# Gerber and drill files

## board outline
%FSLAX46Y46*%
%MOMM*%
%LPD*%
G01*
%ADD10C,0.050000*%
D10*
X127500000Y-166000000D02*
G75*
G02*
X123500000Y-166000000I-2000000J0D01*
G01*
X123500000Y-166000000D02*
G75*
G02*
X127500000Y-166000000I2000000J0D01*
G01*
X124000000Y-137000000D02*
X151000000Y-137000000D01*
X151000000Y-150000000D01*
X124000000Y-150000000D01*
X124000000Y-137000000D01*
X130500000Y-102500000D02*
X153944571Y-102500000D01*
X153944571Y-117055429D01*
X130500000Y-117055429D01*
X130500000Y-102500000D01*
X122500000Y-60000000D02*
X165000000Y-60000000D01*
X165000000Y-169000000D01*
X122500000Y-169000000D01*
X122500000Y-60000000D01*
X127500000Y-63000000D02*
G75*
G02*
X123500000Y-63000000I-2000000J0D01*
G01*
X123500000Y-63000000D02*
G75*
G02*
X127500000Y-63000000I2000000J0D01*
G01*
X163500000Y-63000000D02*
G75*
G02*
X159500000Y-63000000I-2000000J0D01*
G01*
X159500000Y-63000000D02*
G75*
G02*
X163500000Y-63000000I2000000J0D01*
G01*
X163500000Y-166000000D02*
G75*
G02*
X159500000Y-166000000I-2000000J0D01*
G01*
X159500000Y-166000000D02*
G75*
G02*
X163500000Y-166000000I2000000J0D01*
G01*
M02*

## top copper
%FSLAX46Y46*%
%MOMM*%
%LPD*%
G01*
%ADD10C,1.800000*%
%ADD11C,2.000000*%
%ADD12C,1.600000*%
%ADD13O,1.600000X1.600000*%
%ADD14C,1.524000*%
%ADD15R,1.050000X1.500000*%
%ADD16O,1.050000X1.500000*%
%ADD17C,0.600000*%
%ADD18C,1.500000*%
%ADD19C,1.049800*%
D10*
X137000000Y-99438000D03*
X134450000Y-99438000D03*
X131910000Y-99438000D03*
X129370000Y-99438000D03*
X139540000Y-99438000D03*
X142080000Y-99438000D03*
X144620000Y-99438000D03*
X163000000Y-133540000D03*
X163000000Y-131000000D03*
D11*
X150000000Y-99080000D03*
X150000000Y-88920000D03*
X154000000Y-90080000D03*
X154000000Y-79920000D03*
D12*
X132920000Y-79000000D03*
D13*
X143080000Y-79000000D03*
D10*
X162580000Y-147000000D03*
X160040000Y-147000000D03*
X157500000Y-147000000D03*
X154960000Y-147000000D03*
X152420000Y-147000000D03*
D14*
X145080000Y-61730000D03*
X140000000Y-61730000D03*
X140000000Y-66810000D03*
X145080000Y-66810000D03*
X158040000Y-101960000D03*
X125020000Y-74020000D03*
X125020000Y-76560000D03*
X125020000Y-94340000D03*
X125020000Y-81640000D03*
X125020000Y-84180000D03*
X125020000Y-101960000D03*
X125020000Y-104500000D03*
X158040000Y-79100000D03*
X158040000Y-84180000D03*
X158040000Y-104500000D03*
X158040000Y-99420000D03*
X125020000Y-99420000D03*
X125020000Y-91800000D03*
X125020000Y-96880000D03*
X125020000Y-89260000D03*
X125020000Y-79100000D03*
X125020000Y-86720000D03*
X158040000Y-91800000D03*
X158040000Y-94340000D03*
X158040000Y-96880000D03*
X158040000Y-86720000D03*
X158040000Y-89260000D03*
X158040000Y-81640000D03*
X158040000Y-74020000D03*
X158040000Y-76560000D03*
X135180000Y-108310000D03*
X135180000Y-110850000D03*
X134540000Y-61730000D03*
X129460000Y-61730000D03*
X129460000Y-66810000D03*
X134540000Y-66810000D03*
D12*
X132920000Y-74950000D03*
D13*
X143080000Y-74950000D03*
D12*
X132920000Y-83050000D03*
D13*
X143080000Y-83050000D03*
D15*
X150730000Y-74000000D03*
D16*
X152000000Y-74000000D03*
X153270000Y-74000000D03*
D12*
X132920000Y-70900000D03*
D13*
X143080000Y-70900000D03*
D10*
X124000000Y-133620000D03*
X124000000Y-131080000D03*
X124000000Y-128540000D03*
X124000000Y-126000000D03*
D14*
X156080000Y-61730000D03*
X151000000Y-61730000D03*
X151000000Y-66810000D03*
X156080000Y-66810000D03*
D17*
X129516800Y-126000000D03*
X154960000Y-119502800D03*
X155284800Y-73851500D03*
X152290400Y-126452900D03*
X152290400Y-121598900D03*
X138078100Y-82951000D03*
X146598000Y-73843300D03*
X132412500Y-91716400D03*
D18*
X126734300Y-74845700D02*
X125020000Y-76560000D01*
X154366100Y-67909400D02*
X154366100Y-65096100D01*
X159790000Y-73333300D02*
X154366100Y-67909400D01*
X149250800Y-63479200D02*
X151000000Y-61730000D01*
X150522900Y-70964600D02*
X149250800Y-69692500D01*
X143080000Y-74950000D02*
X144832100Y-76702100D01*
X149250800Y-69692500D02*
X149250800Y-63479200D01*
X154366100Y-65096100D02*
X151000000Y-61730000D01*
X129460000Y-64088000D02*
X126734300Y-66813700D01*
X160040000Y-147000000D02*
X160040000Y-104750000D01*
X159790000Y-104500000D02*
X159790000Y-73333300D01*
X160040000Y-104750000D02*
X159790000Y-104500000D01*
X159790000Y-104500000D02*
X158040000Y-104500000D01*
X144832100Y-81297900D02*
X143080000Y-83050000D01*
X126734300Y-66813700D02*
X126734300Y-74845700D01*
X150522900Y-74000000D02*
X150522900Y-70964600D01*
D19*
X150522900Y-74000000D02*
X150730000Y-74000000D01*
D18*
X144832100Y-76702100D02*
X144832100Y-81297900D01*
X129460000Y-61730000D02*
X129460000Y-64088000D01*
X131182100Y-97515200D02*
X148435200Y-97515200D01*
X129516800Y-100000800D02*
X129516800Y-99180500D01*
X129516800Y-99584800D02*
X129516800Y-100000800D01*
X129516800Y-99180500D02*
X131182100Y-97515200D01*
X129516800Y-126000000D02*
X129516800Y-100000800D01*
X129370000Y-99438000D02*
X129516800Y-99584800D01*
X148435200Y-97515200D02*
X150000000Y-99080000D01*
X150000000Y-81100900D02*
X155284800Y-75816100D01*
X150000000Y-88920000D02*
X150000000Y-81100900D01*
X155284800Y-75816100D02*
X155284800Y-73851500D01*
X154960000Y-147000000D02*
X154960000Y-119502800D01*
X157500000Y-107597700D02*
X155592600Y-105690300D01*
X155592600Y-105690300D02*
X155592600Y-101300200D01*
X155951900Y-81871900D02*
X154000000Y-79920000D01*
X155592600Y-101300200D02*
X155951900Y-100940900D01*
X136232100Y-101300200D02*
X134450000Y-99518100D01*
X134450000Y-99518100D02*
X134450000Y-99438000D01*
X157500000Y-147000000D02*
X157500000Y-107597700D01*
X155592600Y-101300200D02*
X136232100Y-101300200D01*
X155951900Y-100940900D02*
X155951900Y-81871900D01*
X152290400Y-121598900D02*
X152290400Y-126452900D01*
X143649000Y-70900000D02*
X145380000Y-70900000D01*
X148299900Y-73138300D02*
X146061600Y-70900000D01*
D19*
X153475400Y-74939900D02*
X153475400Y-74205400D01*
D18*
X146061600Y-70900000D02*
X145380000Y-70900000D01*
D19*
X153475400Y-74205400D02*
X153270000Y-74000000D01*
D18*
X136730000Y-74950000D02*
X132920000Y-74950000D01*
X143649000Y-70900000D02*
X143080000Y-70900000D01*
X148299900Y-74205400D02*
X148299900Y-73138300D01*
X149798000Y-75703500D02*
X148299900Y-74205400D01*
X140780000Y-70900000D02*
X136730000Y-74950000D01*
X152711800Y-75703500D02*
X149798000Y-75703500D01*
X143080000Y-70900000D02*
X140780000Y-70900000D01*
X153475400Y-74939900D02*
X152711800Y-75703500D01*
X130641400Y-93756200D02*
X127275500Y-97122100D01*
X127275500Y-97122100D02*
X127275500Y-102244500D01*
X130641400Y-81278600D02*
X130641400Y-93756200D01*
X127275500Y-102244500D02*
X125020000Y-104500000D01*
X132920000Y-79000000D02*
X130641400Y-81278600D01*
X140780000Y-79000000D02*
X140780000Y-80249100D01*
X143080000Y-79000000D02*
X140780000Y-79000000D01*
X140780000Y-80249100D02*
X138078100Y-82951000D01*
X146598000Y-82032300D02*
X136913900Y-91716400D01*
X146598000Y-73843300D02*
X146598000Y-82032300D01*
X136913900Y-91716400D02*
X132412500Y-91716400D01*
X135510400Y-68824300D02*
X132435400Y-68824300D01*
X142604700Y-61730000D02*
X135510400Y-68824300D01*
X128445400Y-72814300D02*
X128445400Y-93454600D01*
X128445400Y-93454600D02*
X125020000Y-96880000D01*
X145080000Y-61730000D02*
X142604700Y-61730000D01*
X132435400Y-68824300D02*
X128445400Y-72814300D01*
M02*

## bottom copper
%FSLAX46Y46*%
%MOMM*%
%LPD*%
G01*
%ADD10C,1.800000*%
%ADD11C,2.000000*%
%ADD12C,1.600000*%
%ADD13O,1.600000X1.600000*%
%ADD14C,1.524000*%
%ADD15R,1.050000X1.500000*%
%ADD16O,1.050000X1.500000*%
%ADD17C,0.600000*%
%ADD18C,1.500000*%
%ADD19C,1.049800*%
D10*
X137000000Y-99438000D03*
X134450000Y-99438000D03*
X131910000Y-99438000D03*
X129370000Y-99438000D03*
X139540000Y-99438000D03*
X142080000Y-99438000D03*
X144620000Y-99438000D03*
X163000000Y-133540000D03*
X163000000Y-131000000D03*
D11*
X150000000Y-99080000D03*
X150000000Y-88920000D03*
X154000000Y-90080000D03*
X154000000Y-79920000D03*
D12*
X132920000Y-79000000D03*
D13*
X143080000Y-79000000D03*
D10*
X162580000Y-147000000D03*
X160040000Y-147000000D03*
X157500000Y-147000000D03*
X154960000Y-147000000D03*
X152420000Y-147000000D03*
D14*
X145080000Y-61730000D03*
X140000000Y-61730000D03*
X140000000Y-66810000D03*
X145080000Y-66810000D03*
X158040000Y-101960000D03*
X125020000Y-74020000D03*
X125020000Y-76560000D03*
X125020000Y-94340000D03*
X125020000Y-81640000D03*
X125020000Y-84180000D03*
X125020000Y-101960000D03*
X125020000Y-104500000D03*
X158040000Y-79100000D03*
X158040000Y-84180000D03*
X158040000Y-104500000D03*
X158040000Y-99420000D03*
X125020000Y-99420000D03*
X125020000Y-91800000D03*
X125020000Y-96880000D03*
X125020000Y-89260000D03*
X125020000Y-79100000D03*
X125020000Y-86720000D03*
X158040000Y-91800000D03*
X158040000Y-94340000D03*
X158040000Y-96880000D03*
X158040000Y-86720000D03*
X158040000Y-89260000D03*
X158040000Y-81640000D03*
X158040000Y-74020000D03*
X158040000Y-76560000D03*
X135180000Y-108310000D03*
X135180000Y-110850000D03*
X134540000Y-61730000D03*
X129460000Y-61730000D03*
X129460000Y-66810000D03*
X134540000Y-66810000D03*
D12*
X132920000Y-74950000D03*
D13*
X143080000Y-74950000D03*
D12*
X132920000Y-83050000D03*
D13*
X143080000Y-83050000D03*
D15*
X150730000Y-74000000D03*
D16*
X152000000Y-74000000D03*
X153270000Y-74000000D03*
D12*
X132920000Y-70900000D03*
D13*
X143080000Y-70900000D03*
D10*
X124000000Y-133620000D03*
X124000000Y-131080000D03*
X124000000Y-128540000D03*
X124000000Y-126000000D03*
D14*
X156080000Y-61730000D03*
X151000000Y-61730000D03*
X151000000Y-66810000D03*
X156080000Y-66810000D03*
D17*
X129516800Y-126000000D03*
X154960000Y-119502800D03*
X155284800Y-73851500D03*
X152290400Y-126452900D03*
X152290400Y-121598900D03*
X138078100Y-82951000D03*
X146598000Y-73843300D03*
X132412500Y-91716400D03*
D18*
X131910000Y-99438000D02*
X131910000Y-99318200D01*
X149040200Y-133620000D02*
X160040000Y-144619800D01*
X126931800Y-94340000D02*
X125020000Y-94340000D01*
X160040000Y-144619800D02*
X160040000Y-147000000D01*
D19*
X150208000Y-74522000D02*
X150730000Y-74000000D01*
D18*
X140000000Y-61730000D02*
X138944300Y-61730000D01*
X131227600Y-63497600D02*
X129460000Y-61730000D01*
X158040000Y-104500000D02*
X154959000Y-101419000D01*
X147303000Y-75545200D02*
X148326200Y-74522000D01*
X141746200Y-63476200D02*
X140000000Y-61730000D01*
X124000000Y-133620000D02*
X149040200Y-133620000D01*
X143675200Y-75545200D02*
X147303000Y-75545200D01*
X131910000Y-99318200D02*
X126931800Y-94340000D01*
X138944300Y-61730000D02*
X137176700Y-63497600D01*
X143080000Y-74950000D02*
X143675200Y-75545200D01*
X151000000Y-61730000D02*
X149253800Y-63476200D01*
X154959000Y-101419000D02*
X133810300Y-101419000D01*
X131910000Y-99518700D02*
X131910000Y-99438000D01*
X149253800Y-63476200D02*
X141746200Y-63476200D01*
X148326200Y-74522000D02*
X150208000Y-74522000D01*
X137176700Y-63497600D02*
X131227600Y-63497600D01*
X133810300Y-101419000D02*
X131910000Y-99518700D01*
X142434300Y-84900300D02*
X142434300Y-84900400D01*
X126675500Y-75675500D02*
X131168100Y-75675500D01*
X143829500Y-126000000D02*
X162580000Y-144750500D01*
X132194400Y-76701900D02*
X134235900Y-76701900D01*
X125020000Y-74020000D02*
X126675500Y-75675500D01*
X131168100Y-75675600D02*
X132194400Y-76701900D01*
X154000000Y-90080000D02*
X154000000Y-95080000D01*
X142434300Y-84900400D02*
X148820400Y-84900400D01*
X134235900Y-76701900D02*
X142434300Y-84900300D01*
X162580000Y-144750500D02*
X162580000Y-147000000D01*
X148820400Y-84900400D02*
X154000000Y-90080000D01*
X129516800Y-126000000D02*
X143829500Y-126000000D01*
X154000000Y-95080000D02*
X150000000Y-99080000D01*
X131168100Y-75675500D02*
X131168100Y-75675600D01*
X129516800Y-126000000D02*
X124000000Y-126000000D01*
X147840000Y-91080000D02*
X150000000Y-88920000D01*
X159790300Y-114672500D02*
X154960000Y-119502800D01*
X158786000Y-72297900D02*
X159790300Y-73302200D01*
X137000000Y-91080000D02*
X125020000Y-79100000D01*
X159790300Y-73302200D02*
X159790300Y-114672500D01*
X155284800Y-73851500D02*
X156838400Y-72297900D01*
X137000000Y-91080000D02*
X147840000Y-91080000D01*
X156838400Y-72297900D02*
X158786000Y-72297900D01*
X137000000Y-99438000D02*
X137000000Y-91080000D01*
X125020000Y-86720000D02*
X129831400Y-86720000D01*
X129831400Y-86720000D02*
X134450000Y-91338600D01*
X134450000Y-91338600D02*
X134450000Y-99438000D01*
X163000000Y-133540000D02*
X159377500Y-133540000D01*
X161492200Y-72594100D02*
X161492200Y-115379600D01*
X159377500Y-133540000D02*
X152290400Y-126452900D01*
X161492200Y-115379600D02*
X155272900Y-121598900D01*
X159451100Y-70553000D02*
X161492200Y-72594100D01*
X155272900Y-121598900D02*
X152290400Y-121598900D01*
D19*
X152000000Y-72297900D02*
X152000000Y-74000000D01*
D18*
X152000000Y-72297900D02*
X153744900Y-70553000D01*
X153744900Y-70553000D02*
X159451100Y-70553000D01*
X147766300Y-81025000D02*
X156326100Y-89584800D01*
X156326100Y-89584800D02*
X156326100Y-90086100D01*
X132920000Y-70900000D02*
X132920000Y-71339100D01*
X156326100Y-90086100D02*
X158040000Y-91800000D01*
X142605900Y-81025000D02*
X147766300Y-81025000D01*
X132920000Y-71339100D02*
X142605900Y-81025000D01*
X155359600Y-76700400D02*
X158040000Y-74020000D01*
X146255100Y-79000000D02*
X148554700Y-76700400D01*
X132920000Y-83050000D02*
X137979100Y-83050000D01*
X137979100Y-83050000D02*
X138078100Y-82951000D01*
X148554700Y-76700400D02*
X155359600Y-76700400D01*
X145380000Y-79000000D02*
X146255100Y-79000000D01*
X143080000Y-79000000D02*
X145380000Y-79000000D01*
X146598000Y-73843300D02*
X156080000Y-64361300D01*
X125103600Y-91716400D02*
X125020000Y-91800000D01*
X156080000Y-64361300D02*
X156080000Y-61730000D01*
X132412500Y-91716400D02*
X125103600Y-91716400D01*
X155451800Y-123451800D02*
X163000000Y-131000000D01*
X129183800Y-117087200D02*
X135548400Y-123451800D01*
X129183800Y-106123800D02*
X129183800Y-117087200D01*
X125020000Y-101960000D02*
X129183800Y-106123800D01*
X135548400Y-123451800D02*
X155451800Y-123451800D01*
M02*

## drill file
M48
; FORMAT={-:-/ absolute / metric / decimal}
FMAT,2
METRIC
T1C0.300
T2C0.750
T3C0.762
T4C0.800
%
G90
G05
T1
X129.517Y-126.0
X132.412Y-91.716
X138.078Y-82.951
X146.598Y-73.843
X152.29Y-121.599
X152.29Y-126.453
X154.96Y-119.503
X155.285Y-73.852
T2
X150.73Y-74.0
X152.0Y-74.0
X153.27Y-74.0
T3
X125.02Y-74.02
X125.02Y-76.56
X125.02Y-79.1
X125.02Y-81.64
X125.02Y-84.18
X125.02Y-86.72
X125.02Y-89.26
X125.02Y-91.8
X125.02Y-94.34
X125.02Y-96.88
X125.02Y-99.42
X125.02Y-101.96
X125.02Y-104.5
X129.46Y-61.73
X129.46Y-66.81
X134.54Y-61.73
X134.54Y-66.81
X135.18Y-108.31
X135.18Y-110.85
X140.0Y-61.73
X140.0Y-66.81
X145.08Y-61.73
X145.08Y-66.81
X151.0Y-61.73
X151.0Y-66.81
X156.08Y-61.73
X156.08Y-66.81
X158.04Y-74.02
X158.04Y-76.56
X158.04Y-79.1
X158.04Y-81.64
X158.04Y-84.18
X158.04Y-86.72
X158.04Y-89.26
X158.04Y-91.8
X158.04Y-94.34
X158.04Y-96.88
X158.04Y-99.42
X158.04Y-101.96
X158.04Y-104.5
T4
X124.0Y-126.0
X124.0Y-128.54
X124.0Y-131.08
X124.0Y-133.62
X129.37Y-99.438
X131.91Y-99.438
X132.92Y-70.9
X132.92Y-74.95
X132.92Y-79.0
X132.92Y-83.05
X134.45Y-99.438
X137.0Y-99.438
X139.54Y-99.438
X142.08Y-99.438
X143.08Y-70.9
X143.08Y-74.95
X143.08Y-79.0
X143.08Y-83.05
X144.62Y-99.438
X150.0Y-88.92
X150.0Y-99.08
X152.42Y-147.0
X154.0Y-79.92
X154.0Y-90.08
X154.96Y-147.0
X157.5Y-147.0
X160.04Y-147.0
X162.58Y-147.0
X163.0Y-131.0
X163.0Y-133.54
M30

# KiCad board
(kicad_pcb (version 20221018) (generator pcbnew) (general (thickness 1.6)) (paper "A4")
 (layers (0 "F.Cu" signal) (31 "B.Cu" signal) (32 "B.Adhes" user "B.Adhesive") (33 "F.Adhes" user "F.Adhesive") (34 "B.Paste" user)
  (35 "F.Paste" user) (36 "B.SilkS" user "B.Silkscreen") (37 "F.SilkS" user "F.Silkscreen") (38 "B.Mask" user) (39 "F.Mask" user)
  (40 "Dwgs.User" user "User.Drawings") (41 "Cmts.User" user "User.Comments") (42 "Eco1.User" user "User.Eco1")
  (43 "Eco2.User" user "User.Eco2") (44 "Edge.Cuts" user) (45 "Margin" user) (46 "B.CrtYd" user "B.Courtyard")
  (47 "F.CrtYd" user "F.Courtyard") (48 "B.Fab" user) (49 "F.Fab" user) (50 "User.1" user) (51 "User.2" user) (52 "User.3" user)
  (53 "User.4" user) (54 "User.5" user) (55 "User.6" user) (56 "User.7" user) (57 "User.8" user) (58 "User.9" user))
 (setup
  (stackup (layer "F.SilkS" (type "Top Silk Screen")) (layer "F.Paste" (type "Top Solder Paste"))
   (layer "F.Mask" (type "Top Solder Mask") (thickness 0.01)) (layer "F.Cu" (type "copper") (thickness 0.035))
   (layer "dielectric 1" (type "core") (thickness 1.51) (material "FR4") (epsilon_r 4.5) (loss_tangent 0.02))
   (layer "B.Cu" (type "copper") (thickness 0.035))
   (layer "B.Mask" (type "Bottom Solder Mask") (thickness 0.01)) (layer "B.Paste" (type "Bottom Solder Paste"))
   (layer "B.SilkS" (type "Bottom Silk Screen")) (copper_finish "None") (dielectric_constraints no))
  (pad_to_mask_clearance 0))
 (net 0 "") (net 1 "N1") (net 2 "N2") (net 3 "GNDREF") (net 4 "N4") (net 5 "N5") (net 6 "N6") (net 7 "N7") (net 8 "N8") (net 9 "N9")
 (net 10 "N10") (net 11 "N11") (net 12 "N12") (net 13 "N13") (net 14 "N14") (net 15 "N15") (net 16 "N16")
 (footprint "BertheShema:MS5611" (layer "F.Cu") (at 133.19 96.898)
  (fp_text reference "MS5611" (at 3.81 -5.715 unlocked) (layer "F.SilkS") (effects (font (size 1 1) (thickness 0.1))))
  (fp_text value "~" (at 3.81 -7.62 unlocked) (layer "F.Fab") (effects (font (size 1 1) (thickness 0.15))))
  (pad "1" thru_hole circle (at 3.81 2.54) (size 1.8 1.8) (drill 0.8) (layers "*.Cu" "*.Mask") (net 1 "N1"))
  (pad "2" thru_hole circle (at 1.26 2.54) (size 1.8 1.8) (drill 0.8) (layers "*.Cu" "*.Mask") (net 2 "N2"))
  (pad "3" thru_hole circle (at -1.28 2.54) (size 1.8 1.8) (drill 0.8) (layers "*.Cu" "*.Mask") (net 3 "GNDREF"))
  (pad "4" thru_hole circle (at -3.82 2.54) (size 1.8 1.8) (drill 0.8) (layers "*.Cu" "*.Mask") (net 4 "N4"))
  (pad "5" thru_hole circle (at 6.35 2.54) (size 1.8 1.8) (drill 0.8) (layers "*.Cu" "*.Mask"))
  (pad "6" thru_hole circle (at 8.89 2.54) (size 1.8 1.8) (drill 0.8) (layers "*.Cu" "*.Mask"))
  (pad "7" thru_hole circle (at 11.43 2.54) (size 1.8 1.8) (drill 0.8) (layers "*.Cu" "*.Mask")))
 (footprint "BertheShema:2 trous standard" (layer "F.Cu") (at 163 133.54)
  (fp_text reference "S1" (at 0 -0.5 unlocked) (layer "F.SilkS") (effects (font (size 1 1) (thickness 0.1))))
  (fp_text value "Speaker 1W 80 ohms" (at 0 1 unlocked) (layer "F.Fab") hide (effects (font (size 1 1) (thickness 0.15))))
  (pad "1" thru_hole circle (at 0 0) (size 1.8 1.8) (drill 0.8) (layers "*.Cu" "*.Mask") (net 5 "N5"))
  (pad "2" thru_hole circle (at 0 -2.54) (size 1.8 1.8) (drill 0.8) (layers "*.Cu" "*.Mask") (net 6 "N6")))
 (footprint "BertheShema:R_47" (layer "F.Cu") (at 150 94 -90)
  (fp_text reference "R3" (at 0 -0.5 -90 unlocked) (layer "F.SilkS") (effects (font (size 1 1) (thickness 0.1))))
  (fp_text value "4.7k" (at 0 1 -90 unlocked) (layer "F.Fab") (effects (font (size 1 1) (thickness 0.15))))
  (pad "1" thru_hole circle (at 5.08 0 270) (size 2 2) (drill 0.8) (layers "*.Cu" "*.Mask") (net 4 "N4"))
  (pad "2" thru_hole circle (at -5.08 0 270) (size 2 2) (drill 0.8) (layers "*.Cu" "*.Mask") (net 1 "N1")))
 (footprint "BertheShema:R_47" (layer "F.Cu") (at 154 85 -90)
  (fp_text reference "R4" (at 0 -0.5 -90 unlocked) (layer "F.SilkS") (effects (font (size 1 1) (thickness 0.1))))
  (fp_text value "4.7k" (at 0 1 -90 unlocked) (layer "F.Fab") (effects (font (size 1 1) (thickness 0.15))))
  (pad "1" thru_hole circle (at 5.08 0 270) (size 2 2) (drill 0.8) (layers "*.Cu" "*.Mask") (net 4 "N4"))
  (pad "2" thru_hole circle (at -5.08 0 270) (size 2 2) (drill 0.8) (layers "*.Cu" "*.Mask") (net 2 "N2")))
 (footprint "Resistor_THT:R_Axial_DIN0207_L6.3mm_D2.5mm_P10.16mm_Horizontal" (layer "F.Cu") (at 132.92 79)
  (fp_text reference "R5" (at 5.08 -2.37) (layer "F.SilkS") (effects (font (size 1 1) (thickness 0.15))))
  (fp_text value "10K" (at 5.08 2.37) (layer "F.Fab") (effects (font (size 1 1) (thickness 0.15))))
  (pad "1" thru_hole circle (at 0 0) (size 1.6 1.6) (drill 0.8) (layers "*.Cu" "*.Mask") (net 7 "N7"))
  (pad "2" thru_hole oval (at 10.16 0) (size 1.6 1.6) (drill 0.8) (layers "*.Cu" "*.Mask") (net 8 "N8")))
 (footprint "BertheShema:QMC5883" (layer "F.Cu") (at 157.54 153 180)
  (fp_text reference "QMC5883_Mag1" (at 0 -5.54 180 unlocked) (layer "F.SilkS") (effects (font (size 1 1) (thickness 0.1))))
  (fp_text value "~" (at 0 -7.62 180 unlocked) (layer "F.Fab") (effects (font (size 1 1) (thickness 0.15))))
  (pad "1" thru_hole circle (at -5.04 6 180) (size 1.8 1.8) (drill 0.8) (layers "*.Cu" "*.Mask") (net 4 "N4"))
  (pad "2" thru_hole circle (at -2.5 6 180) (size 1.8 1.8) (drill 0.8) (layers "*.Cu" "*.Mask") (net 3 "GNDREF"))
  (pad "3" thru_hole circle (at 0.04 6 180) (size 1.8 1.8) (drill 0.8) (layers "*.Cu" "*.Mask") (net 2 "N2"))
  (pad "4" thru_hole circle (at 2.58 6 180) (size 1.8 1.8) (drill 0.8) (layers "*.Cu" "*.Mask") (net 1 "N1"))
  (pad "5" thru_hole circle (at 5.12 6 180) (size 1.8 1.8) (drill 0.8) (layers "*.Cu" "*.Mask")))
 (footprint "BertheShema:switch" (layer "F.Cu") (at 142.54 63)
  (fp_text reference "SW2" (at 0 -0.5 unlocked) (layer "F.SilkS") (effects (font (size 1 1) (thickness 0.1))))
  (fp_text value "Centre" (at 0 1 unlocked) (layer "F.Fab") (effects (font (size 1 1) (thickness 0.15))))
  (pad "1" thru_hole circle (at 2.54 -1.27) (size 1.524 1.524) (drill 0.762) (layers "*.Cu" "*.Mask") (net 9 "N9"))
  (pad "2" thru_hole circle (at -2.54 -1.27) (size 1.524 1.524) (drill 0.762) (layers "*.Cu" "*.Mask") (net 3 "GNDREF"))
  (pad "3" thru_hole circle (at -2.54 3.81) (size 1.524 1.524) (drill 0.762) (layers "*.Cu" "*.Mask"))
  (pad "4" thru_hole circle (at 2.54 3.81) (size 1.524 1.524) (drill 0.762) (layers "*.Cu" "*.Mask")))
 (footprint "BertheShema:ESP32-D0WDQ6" (layer "F.Cu") (at 140.26 89.26)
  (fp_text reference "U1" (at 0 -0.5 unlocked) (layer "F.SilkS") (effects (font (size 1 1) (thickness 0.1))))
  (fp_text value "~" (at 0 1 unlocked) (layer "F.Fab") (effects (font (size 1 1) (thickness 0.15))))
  (pad "0" thru_hole circle (at 17.78 12.7) (size 1.524 1.524) (drill 0.762) (layers "*.Cu" "*.Mask"))
  (pad "1" thru_hole circle (at -15.24 -15.24) (size 1.524 1.524) (drill 0.762) (layers "*.Cu" "*.Mask") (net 4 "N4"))
  (pad "2" thru_hole circle (at -15.24 -12.7) (size 1.524 1.524) (drill 0.762) (layers "*.Cu" "*.Mask") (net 3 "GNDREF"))
  (pad "2" thru_hole circle (at -15.24 5.08) (size 1.524 1.524) (drill 0.762) (layers "*.Cu" "*.Mask") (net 3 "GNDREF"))
  (pad "3" thru_hole circle (at -15.24 -7.62) (size 1.524 1.524) (drill 0.762) (layers "*.Cu" "*.Mask") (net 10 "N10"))
  (pad "4" thru_hole circle (at -15.24 -5.08) (size 1.524 1.524) (drill 0.762) (layers "*.Cu" "*.Mask") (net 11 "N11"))
  (pad "5" thru_hole circle (at -15.24 12.7) (size 1.524 1.524) (drill 0.762) (layers "*.Cu" "*.Mask") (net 6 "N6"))
  (pad "6" thru_hole circle (at -15.24 15.24) (size 1.524 1.524) (drill 0.762) (layers "*.Cu" "*.Mask") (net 7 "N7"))
  (pad "7" thru_hole circle (at 17.78 -10.16) (size 1.524 1.524) (drill 0.762) (layers "*.Cu" "*.Mask"))
  (pad "8" thru_hole circle (at 17.78 -5.08) (size 1.524 1.524) (drill 0.762) (layers "*.Cu" "*.Mask"))
  (pad "9" thru_hole circle (at 17.78 15.24) (size 1.524 1.524) (drill 0.762) (layers "*.Cu" "*.Mask") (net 3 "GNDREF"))
  (pad "12" thru_hole circle (at 17.78 10.16) (size 1.524 1.524) (drill 0.762) (layers "*.Cu" "*.Mask"))
  (pad "13" thru_hole circle (at -15.24 10.16) (size 1.524 1.524) (drill 0.762) (layers "*.Cu" "*.Mask") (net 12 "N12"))
  (pad "14" thru_hole circle (at -15.24 2.54) (size 1.524 1.524) (drill 0.762) (layers "*.Cu" "*.Mask") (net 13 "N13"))
  (pad "15" thru_hole circle (at -15.24 7.62) (size 1.524 1.524) (drill 0.762) (layers "*.Cu" "*.Mask") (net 9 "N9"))
  (pad "19" thru_hole circle (at -15.24 0) (size 1.524 1.524) (drill 0.762) (layers "*.Cu" "*.Mask"))
  (pad "21" thru_hole circle (at -15.24 -10.16) (size 1.524 1.524) (drill 0.762) (layers "*.Cu" "*.Mask") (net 1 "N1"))
  (pad "22" thru_hole circle (at -15.24 -2.54) (size 1.524 1.524) (drill 0.762) (layers "*.Cu" "*.Mask") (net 2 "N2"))
  (pad "25" thru_hole circle (at 17.78 2.54) (size 1.524 1.524) (drill 0.762) (layers "*.Cu" "*.Mask") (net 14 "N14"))
  (pad "26" thru_hole circle (at 17.78 5.08) (size 1.524 1.524) (drill 0.762) (layers "*.Cu" "*.Mask"))
  (pad "27" thru_hole circle (at 17.78 7.62) (size 1.524 1.524) (drill 0.762) (layers "*.Cu" "*.Mask"))
  (pad "32" thru_hole circle (at 17.78 -2.54) (size 1.524 1.524) (drill 0.762) (layers "*.Cu" "*.Mask"))
  (pad "33" thru_hole circle (at 17.78 0) (size 1.524 1.524) (drill 0.762) (layers "*.Cu" "*.Mask"))
  (pad "34" thru_hole circle (at 17.78 -7.62) (size 1.524 1.524) (drill 0.762) (layers "*.Cu" "*.Mask"))
  (pad "36" thru_hole circle (at 17.78 -15.24) (size 1.524 1.524) (drill 0.762) (layers "*.Cu" "*.Mask") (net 8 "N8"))
  (pad "39" thru_hole circle (at 17.78 -12.7) (size 1.524 1.524) (drill 0.762) (layers "*.Cu" "*.Mask"))
  (pad "40" thru_hole circle (at -5.08 19.05) (size 1.524 1.524) (drill 0.762) (layers "*.Cu" "*.Mask"))
  (pad "41" thru_hole circle (at -5.08 21.59) (size 1.524 1.524) (drill 0.762) (layers "*.Cu" "*.Mask")))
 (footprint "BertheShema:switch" (layer "F.Cu") (at 132 63)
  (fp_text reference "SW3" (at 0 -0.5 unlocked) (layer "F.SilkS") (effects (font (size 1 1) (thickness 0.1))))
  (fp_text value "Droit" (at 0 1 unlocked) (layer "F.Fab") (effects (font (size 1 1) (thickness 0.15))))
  (pad "1" thru_hole circle (at 2.54 -1.27) (size 1.524 1.524) (drill 0.762) (layers "*.Cu" "*.Mask") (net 12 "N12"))
  (pad "2" thru_hole circle (at -2.54 -1.27) (size 1.524 1.524) (drill 0.762) (layers "*.Cu" "*.Mask") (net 3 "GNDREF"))
  (pad "3" thru_hole circle (at -2.54 3.81) (size 1.524 1.524) (drill 0.762) (layers "*.Cu" "*.Mask"))
  (pad "4" thru_hole circle (at 2.54 3.81) (size 1.524 1.524) (drill 0.762) (layers "*.Cu" "*.Mask")))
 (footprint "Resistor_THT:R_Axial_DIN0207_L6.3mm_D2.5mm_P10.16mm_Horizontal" (layer "F.Cu") (at 132.92 74.95)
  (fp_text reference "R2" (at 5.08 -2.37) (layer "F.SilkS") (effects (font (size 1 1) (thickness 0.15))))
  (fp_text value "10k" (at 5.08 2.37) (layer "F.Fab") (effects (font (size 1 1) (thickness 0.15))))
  (pad "1" thru_hole circle (at 0 0) (size 1.6 1.6) (drill 0.8) (layers "*.Cu" "*.Mask") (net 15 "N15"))
  (pad "2" thru_hole oval (at 10.16 0) (size 1.6 1.6) (drill 0.8) (layers "*.Cu" "*.Mask") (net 3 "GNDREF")))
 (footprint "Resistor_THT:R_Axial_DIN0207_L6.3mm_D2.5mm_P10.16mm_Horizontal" (layer "F.Cu") (at 132.92 83.05)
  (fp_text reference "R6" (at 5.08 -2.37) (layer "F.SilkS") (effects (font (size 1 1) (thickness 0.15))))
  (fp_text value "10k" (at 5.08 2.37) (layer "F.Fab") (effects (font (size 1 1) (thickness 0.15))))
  (pad "1" thru_hole circle (at 0 0) (size 1.6 1.6) (drill 0.8) (layers "*.Cu" "*.Mask") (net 8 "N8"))
  (pad "2" thru_hole oval (at 10.16 0) (size 1.6 1.6) (drill 0.8) (layers "*.Cu" "*.Mask") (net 3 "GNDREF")))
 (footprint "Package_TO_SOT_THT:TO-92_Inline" (layer "F.Cu") (at 150.73 74)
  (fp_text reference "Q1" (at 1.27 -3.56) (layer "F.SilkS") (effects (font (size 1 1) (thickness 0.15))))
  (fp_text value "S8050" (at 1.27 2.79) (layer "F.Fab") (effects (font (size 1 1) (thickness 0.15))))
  (pad "1" thru_hole rect (at 0 0) (size 1.05 1.5) (drill 0.75) (layers "*.Cu" "*.Mask") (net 3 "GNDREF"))
  (pad "2" thru_hole oval (at 1.27 0) (size 1.05 1.5) (drill 0.75) (layers "*.Cu" "*.Mask") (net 5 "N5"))
  (pad "3" thru_hole oval (at 2.54 0) (size 1.05 1.5) (drill 0.75) (layers "*.Cu" "*.Mask") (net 15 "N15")))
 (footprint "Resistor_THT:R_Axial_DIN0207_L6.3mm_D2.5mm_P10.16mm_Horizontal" (layer "F.Cu") (at 132.92 70.9)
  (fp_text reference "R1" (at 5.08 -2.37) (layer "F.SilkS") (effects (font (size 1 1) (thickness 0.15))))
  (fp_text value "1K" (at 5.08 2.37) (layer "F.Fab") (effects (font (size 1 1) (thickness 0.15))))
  (pad "1" thru_hole circle (at 0 0) (size 1.6 1.6) (drill 0.8) (layers "*.Cu" "*.Mask") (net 14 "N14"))
  (pad "2" thru_hole oval (at 10.16 0) (size 1.6 1.6) (drill 0.8) (layers "*.Cu" "*.Mask") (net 15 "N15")))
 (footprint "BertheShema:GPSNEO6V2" (layer "F.Cu") (at 125.905 129.81 -90)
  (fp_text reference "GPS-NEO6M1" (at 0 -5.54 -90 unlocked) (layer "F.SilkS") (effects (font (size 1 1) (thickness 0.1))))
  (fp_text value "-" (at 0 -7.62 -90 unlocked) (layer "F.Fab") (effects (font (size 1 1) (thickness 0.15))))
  (pad "1" thru_hole circle (at 3.81 1.905 270) (size 1.8 1.8) (drill 0.8) (layers "*.Cu" "*.Mask") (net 3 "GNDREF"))
  (pad "2" thru_hole circle (at 1.27 1.905 270) (size 1.8 1.8) (drill 0.8) (layers "*.Cu" "*.Mask") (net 10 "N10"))
  (pad "3" thru_hole circle (at -1.27 1.905 270) (size 1.8 1.8) (drill 0.8) (layers "*.Cu" "*.Mask") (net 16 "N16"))
  (pad "4" thru_hole circle (at -3.81 1.905 270) (size 1.8 1.8) (drill 0.8) (layers "*.Cu" "*.Mask") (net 4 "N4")))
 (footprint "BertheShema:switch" (layer "F.Cu") (at 153.54 63)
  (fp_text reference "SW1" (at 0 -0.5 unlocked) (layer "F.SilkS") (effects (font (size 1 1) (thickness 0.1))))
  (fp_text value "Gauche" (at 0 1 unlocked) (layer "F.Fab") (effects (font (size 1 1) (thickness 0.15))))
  (pad "1" thru_hole circle (at 2.54 -1.27) (size 1.524 1.524) (drill 0.762) (layers "*.Cu" "*.Mask") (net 13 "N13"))
  (pad "2" thru_hole circle (at -2.54 -1.27) (size 1.524 1.524) (drill 0.762) (layers "*.Cu" "*.Mask") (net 3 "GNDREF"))
  (pad "3" thru_hole circle (at -2.54 3.81) (size 1.524 1.524) (drill 0.762) (layers "*.Cu" "*.Mask"))
  (pad "4" thru_hole circle (at 2.54 3.81) (size 1.524 1.524) (drill 0.762) (layers "*.Cu" "*.Mask")))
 (gr_circle (center 125.5 166) (end 127.5 166) (stroke (width 0.05) (type default)) (fill none) (layer "Edge.Cuts"))
 (gr_rect (start 124 137) (end 151 150) (stroke (width 0.05) (type default)) (fill none) (layer "Edge.Cuts"))
 (gr_rect (start 130.5 102.5) (end 153.944571 117.055429) (stroke (width 0.05) (type default)) (fill none) (layer "Edge.Cuts"))
 (gr_rect (start 122.5 60) (end 165 169) (stroke (width 0.05) (type default)) (fill none) (layer "Edge.Cuts"))
 (gr_circle (center 125.5 63) (end 127.5 63) (stroke (width 0.05) (type default)) (fill none) (layer "Edge.Cuts"))
 (gr_circle (center 161.5 63) (end 163.5 63) (stroke (width 0.05) (type default)) (fill none) (layer "Edge.Cuts"))
 (gr_rect (start 137 165) (end 137 165) (stroke (width 0.05) (type default)) (fill none) (layer "Edge.Cuts"))
 (gr_circle (center 161.5 166) (end 163.5 166) (stroke (width 0.05) (type default)) (fill none) (layer "Edge.Cuts"))
 (segment (start 126.7343 74.8457) (end 125.02 76.56) (width 1.5) (layer "F.Cu") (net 3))
 (segment (start 154.3661 67.9094) (end 154.3661 65.0961) (width 1.5) (layer "F.Cu") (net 3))
 (segment (start 159.79 73.3333) (end 154.3661 67.9094) (width 1.5) (layer "F.Cu") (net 3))
 (segment (start 149.2508 63.4792) (end 151 61.73) (width 1.5) (layer "F.Cu") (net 3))
 (segment (start 150.5229 70.9646) (end 149.2508 69.6925) (width 1.5) (layer "F.Cu") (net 3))
 (segment (start 143.08 74.95) (end 144.8321 76.7021) (width 1.5) (layer "F.Cu") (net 3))
 (segment (start 149.2508 69.6925) (end 149.2508 63.4792) (width 1.5) (layer "F.Cu") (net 3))
 (segment (start 154.3661 65.0961) (end 151 61.73) (width 1.5) (layer "F.Cu") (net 3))
 (segment (start 129.46 64.088) (end 126.7343 66.8137) (width 1.5) (layer "F.Cu") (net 3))
 (segment (start 160.04 147) (end 160.04 104.75) (width 1.5) (layer "F.Cu") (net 3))
 (segment (start 159.79 104.5) (end 159.79 73.3333) (width 1.5) (layer "F.Cu") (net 3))
 (segment (start 160.04 104.75) (end 159.79 104.5) (width 1.5) (layer "F.Cu") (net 3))
 (segment (start 159.79 104.5) (end 158.04 104.5) (width 1.5) (layer "F.Cu") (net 3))
 (segment (start 144.8321 81.2979) (end 143.08 83.05) (width 1.5) (layer "F.Cu") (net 3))
 (segment (start 126.7343 66.8137) (end 126.7343 74.8457) (width 1.5) (layer "F.Cu") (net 3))
 (segment (start 150.5229 74) (end 150.5229 70.9646) (width 1.5) (layer "F.Cu") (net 3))
 (segment (start 150.5229 74) (end 150.73 74) (width 1.0498) (layer "F.Cu") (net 3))
 (segment (start 144.8321 76.7021) (end 144.8321 81.2979) (width 1.5) (layer "F.Cu") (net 3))
 (segment (start 129.46 61.73) (end 129.46 64.088) (width 1.5) (layer "F.Cu") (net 3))
 (segment (start 131.91 99.438) (end 131.91 99.3182) (width 1.5) (layer "B.Cu") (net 3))
 (segment (start 149.0402 133.62) (end 160.04 144.6198) (width 1.5) (layer "B.Cu") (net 3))
 (segment (start 126.9318 94.34) (end 125.02 94.34) (width 1.5) (layer "B.Cu") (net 3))
 (segment (start 160.04 144.6198) (end 160.04 147) (width 1.5) (layer "B.Cu") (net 3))
 (segment (start 150.208 74.522) (end 150.73 74) (width 1.0498) (layer "B.Cu") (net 3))
 (segment (start 140 61.73) (end 138.9443 61.73) (width 1.5) (layer "B.Cu") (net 3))
 (segment (start 131.2276 63.4976) (end 129.46 61.73) (width 1.5) (layer "B.Cu") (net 3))
 (segment (start 158.04 104.5) (end 154.959 101.419) (width 1.5) (layer "B.Cu") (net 3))
 (segment (start 147.303 75.5452) (end 148.3262 74.522) (width 1.5) (layer "B.Cu") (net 3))
 (segment (start 141.7462 63.4762) (end 140 61.73) (width 1.5) (layer "B.Cu") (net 3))
 (segment (start 124 133.62) (end 149.0402 133.62) (width 1.5) (layer "B.Cu") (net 3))
 (segment (start 143.6752 75.5452) (end 147.303 75.5452) (width 1.5) (layer "B.Cu") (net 3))
 (segment (start 131.91 99.3182) (end 126.9318 94.34) (width 1.5) (layer "B.Cu") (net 3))
 (segment (start 138.9443 61.73) (end 137.1767 63.4976) (width 1.5) (layer "B.Cu") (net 3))
 (segment (start 143.08 74.95) (end 143.6752 75.5452) (width 1.5) (layer "B.Cu") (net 3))
 (segment (start 151 61.73) (end 149.2538 63.4762) (width 1.5) (layer "B.Cu") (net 3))
 (segment (start 154.959 101.419) (end 133.8103 101.419) (width 1.5) (layer "B.Cu") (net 3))
 (segment (start 131.91 99.5187) (end 131.91 99.438) (width 1.5) (layer "B.Cu") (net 3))
 (segment (start 149.2538 63.4762) (end 141.7462 63.4762) (width 1.5) (layer "B.Cu") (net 3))
 (segment (start 148.3262 74.522) (end 150.208 74.522) (width 1.5) (layer "B.Cu") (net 3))
 (segment (start 137.1767 63.4976) (end 131.2276 63.4976) (width 1.5) (layer "B.Cu") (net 3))
 (segment (start 133.8103 101.419) (end 131.91 99.5187) (width 1.5) (layer "B.Cu") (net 3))
 (segment (start 131.1821 97.5152) (end 148.4352 97.5152) (width 1.5) (layer "F.Cu") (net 4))
 (segment (start 129.5168 100.0008) (end 129.5168 99.1805) (width 1.5) (layer "F.Cu") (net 4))
 (segment (start 129.5168 99.5848) (end 129.5168 100.0008) (width 1.5) (layer "F.Cu") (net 4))
 (segment (start 129.5168 99.1805) (end 131.1821 97.5152) (width 1.5) (layer "F.Cu") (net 4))
 (segment (start 129.5168 126) (end 129.5168 100.0008) (width 1.5) (layer "F.Cu") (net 4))
 (segment (start 129.37 99.438) (end 129.5168 99.5848) (width 1.5) (layer "F.Cu") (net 4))
 (segment (start 148.4352 97.5152) (end 150 99.08) (width 1.5) (layer "F.Cu") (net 4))
 (via (at 129.5168 126) (size 0.6) (drill 0.3) (layers "F.Cu" "B.Cu") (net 4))
 (segment (start 142.4343 84.9003) (end 142.4343 84.9004) (width 1.5) (layer "B.Cu") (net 4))
 (segment (start 126.6755 75.6755) (end 131.1681 75.6755) (width 1.5) (layer "B.Cu") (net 4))
 (segment (start 143.8295 126) (end 162.58 144.7505) (width 1.5) (layer "B.Cu") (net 4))
 (segment (start 132.1944 76.7019) (end 134.2359 76.7019) (width 1.5) (layer "B.Cu") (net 4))
 (segment (start 125.02 74.02) (end 126.6755 75.6755) (width 1.5) (layer "B.Cu") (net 4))
 (segment (start 131.1681 75.6756) (end 132.1944 76.7019) (width 1.5) (layer "B.Cu") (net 4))
 (segment (start 154 90.08) (end 154 95.08) (width 1.5) (layer "B.Cu") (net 4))
 (segment (start 142.4343 84.9004) (end 148.8204 84.9004) (width 1.5) (layer "B.Cu") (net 4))
 (segment (start 134.2359 76.7019) (end 142.4343 84.9003) (width 1.5) (layer "B.Cu") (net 4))
 (segment (start 162.58 144.7505) (end 162.58 147) (width 1.5) (layer "B.Cu") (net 4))
 (segment (start 148.8204 84.9004) (end 154 90.08) (width 1.5) (layer "B.Cu") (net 4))
 (segment (start 129.5168 126) (end 143.8295 126) (width 1.5) (layer "B.Cu") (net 4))
 (segment (start 154 95.08) (end 150 99.08) (width 1.5) (layer "B.Cu") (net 4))
 (segment (start 131.1681 75.6755) (end 131.1681 75.6756) (width 1.5) (layer "B.Cu") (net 4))
 (segment (start 129.5168 126) (end 124 126) (width 1.5) (layer "B.Cu") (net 4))
 (segment (start 150 81.1009) (end 155.2848 75.8161) (width 1.5) (layer "F.Cu") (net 1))
 (segment (start 150 88.92) (end 150 81.1009) (width 1.5) (layer "F.Cu") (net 1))
 (segment (start 155.2848 75.8161) (end 155.2848 73.8515) (width 1.5) (layer "F.Cu") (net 1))
 (segment (start 154.96 147) (end 154.96 119.5028) (width 1.5) (layer "F.Cu") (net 1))
 (via (at 154.96 119.5028) (size 0.6) (drill 0.3) (layers "F.Cu" "B.Cu") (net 1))
 (via (at 155.2848 73.8515) (size 0.6) (drill 0.3) (layers "F.Cu" "B.Cu") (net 1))
 (segment (start 147.84 91.08) (end 150 88.92) (width 1.5) (layer "B.Cu") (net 1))
 (segment (start 159.7903 114.6725) (end 154.96 119.5028) (width 1.5) (layer "B.Cu") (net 1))
 (segment (start 158.786 72.2979) (end 159.7903 73.3022) (width 1.5) (layer "B.Cu") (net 1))
 (segment (start 137 91.08) (end 125.02 79.1) (width 1.5) (layer "B.Cu") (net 1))
 (segment (start 159.7903 73.3022) (end 159.7903 114.6725) (width 1.5) (layer "B.Cu") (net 1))
 (segment (start 155.2848 73.8515) (end 156.8384 72.2979) (width 1.5) (layer "B.Cu") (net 1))
 (segment (start 137 91.08) (end 147.84 91.08) (width 1.5) (layer "B.Cu") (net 1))
 (segment (start 156.8384 72.2979) (end 158.786 72.2979) (width 1.5) (layer "B.Cu") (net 1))
 (segment (start 137 99.438) (end 137 91.08) (width 1.5) (layer "B.Cu") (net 1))
 (segment (start 157.5 107.5977) (end 155.5926 105.6903) (width 1.5) (layer "F.Cu") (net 2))
 (segment (start 155.5926 105.6903) (end 155.5926 101.3002) (width 1.5) (layer "F.Cu") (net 2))
 (segment (start 155.9519 81.8719) (end 154 79.92) (width 1.5) (layer "F.Cu") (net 2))
 (segment (start 155.5926 101.3002) (end 155.9519 100.9409) (width 1.5) (layer "F.Cu") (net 2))
 (segment (start 136.2321 101.3002) (end 134.45 99.5181) (width 1.5) (layer "F.Cu") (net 2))
 (segment (start 134.45 99.5181) (end 134.45 99.438) (width 1.5) (layer "F.Cu") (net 2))
 (segment (start 157.5 147) (end 157.5 107.5977) (width 1.5) (layer "F.Cu") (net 2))
 (segment (start 155.5926 101.3002) (end 136.2321 101.3002) (width 1.5) (layer "F.Cu") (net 2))
 (segment (start 155.9519 100.9409) (end 155.9519 81.8719) (width 1.5) (layer "F.Cu") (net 2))
 (segment (start 125.02 86.72) (end 129.8314 86.72) (width 1.5) (layer "B.Cu") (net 2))
 (segment (start 129.8314 86.72) (end 134.45 91.3386) (width 1.5) (layer "B.Cu") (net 2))
 (segment (start 134.45 91.3386) (end 134.45 99.438) (width 1.5) (layer "B.Cu") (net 2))
 (segment (start 152.2904 121.5989) (end 152.2904 126.4529) (width 1.5) (layer "F.Cu") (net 5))
 (via (at 152.2904 126.4529) (size 0.6) (drill 0.3) (layers "F.Cu" "B.Cu") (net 5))
 (via (at 152.2904 121.5989) (size 0.6) (drill 0.3) (layers "F.Cu" "B.Cu") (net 5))
 (segment (start 163 133.54) (end 159.3775 133.54) (width 1.5) (layer "B.Cu") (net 5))
 (segment (start 161.4922 72.5941) (end 161.4922 115.3796) (width 1.5) (layer "B.Cu") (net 5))
 (segment (start 159.3775 133.54) (end 152.2904 126.4529) (width 1.5) (layer "B.Cu") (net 5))
 (segment (start 161.4922 115.3796) (end 155.2729 121.5989) (width 1.5) (layer "B.Cu") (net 5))
 (segment (start 159.4511 70.553) (end 161.4922 72.5941) (width 1.5) (layer "B.Cu") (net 5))
 (segment (start 155.2729 121.5989) (end 152.2904 121.5989) (width 1.5) (layer "B.Cu") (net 5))
 (segment (start 152 72.2979) (end 152 74) (width 1.0498) (layer "B.Cu") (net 5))
 (segment (start 152 72.2979) (end 153.7449 70.553) (width 1.5) (layer "B.Cu") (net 5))
 (segment (start 153.7449 70.553) (end 159.4511 70.553) (width 1.5) (layer "B.Cu") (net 5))
 (segment (start 143.649 70.9) (end 145.38 70.9) (width 1.5) (layer "F.Cu") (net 15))
 (segment (start 148.2999 73.1383) (end 146.0616 70.9) (width 1.5) (layer "F.Cu") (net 15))
 (segment (start 153.4754 74.9399) (end 153.4754 74.2054) (width 1.0498) (layer "F.Cu") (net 15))
 (segment (start 146.0616 70.9) (end 145.38 70.9) (width 1.5) (layer "F.Cu") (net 15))
 (segment (start 153.4754 74.2054) (end 153.27 74) (width 1.0498) (layer "F.Cu") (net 15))
 (segment (start 136.73 74.95) (end 132.92 74.95) (width 1.5) (layer "F.Cu") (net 15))
 (segment (start 143.649 70.9) (end 143.08 70.9) (width 1.5) (layer "F.Cu") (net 15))
 (segment (start 148.2999 74.2054) (end 148.2999 73.1383) (width 1.5) (layer "F.Cu") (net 15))
 (segment (start 149.798 75.7035) (end 148.2999 74.2054) (width 1.5) (layer "F.Cu") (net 15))
 (segment (start 140.78 70.9) (end 136.73 74.95) (width 1.5) (layer "F.Cu") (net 15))
 (segment (start 152.7118 75.7035) (end 149.798 75.7035) (width 1.5) (layer "F.Cu") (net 15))
 (segment (start 143.08 70.9) (end 140.78 70.9) (width 1.5) (layer "F.Cu") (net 15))
 (segment (start 153.4754 74.9399) (end 152.7118 75.7035) (width 1.5) (layer "F.Cu") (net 15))
 (segment (start 147.7663 81.025) (end 156.3261 89.5848) (width 1.5) (layer "B.Cu") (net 14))
 (segment (start 156.3261 89.5848) (end 156.3261 90.0861) (width 1.5) (layer "B.Cu") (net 14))
 (segment (start 132.92 70.9) (end 132.92 71.3391) (width 1.5) (layer "B.Cu") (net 14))
 (segment (start 156.3261 90.0861) (end 158.04 91.8) (width 1.5) (layer "B.Cu") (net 14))
 (segment (start 142.6059 81.025) (end 147.7663 81.025) (width 1.5) (layer "B.Cu") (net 14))
 (segment (start 132.92 71.3391) (end 142.6059 81.025) (width 1.5) (layer "B.Cu") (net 14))
 (segment (start 130.6414 93.7562) (end 127.2755 97.1221) (width 1.5) (layer "F.Cu") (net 7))
 (segment (start 127.2755 97.1221) (end 127.2755 102.2445) (width 1.5) (layer "F.Cu") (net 7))
 (segment (start 130.6414 81.2786) (end 130.6414 93.7562) (width 1.5) (layer "F.Cu") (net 7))
 (segment (start 127.2755 102.2445) (end 125.02 104.5) (width 1.5) (layer "F.Cu") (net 7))
 (segment (start 132.92 79) (end 130.6414 81.2786) (width 1.5) (layer "F.Cu") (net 7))
 (segment (start 140.78 79) (end 140.78 80.2491) (width 1.5) (layer "F.Cu") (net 8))
 (segment (start 143.08 79) (end 140.78 79) (width 1.5) (layer "F.Cu") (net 8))
 (segment (start 140.78 80.2491) (end 138.0781 82.951) (width 1.5) (layer "F.Cu") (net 8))
 (via (at 138.0781 82.951) (size 0.6) (drill 0.3) (layers "F.Cu" "B.Cu") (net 8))
 (segment (start 155.3596 76.7004) (end 158.04 74.02) (width 1.5) (layer "B.Cu") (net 8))
 (segment (start 146.2551 79) (end 148.5547 76.7004) (width 1.5) (layer "B.Cu") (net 8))
 (segment (start 132.92 83.05) (end 137.9791 83.05) (width 1.5) (layer "B.Cu") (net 8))
 (segment (start 137.9791 83.05) (end 138.0781 82.951) (width 1.5) (layer "B.Cu") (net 8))
 (segment (start 148.5547 76.7004) (end 155.3596 76.7004) (width 1.5) (layer "B.Cu") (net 8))
 (segment (start 145.38 79) (end 146.2551 79) (width 1.5) (layer "B.Cu") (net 8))
 (segment (start 143.08 79) (end 145.38 79) (width 1.5) (layer "B.Cu") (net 8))
 (segment (start 146.598 82.0323) (end 136.9139 91.7164) (width 1.5) (layer "F.Cu") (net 13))
 (segment (start 146.598 73.8433) (end 146.598 82.0323) (width 1.5) (layer "F.Cu") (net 13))
 (segment (start 136.9139 91.7164) (end 132.4125 91.7164) (width 1.5) (layer "F.Cu") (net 13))
 (via (at 146.598 73.8433) (size 0.6) (drill 0.3) (layers "F.Cu" "B.Cu") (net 13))
 (via (at 132.4125 91.7164) (size 0.6) (drill 0.3) (layers "F.Cu" "B.Cu") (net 13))
 (segment (start 146.598 73.8433) (end 156.08 64.3613) (width 1.5) (layer "B.Cu") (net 13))
 (segment (start 125.1036 91.7164) (end 125.02 91.8) (width 1.5) (layer "B.Cu") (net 13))
 (segment (start 156.08 64.3613) (end 156.08 61.73) (width 1.5) (layer "B.Cu") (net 13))
 (segment (start 132.4125 91.7164) (end 125.1036 91.7164) (width 1.5) (layer "B.Cu") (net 13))
 (segment (start 135.5104 68.8243) (end 132.4354 68.8243) (width 1.5) (layer "F.Cu") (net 9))
 (segment (start 142.6047 61.73) (end 135.5104 68.8243) (width 1.5) (layer "F.Cu") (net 9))
 (segment (start 128.4454 72.8143) (end 128.4454 93.4546) (width 1.5) (layer "F.Cu") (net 9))
 (segment (start 128.4454 93.4546) (end 125.02 96.88) (width 1.5) (layer "F.Cu") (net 9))
 (segment (start 145.08 61.73) (end 142.6047 61.73) (width 1.5) (layer "F.Cu") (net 9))
 (segment (start 132.4354 68.8243) (end 128.4454 72.8143) (width 1.5) (layer "F.Cu") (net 9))
 (segment (start 155.4518 123.4518) (end 163 131) (width 1.5) (layer "B.Cu") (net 6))
 (segment (start 129.1838 117.0872) (end 135.5484 123.4518) (width 1.5) (layer "B.Cu") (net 6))
 (segment (start 129.1838 106.1238) (end 129.1838 117.0872) (width 1.5) (layer "B.Cu") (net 6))
 (segment (start 125.02 101.96) (end 129.1838 106.1238) (width 1.5) (layer "B.Cu") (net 6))
 (segment (start 135.5484 123.4518) (end 155.4518 123.4518) (width 1.5) (layer "B.Cu") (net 6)))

